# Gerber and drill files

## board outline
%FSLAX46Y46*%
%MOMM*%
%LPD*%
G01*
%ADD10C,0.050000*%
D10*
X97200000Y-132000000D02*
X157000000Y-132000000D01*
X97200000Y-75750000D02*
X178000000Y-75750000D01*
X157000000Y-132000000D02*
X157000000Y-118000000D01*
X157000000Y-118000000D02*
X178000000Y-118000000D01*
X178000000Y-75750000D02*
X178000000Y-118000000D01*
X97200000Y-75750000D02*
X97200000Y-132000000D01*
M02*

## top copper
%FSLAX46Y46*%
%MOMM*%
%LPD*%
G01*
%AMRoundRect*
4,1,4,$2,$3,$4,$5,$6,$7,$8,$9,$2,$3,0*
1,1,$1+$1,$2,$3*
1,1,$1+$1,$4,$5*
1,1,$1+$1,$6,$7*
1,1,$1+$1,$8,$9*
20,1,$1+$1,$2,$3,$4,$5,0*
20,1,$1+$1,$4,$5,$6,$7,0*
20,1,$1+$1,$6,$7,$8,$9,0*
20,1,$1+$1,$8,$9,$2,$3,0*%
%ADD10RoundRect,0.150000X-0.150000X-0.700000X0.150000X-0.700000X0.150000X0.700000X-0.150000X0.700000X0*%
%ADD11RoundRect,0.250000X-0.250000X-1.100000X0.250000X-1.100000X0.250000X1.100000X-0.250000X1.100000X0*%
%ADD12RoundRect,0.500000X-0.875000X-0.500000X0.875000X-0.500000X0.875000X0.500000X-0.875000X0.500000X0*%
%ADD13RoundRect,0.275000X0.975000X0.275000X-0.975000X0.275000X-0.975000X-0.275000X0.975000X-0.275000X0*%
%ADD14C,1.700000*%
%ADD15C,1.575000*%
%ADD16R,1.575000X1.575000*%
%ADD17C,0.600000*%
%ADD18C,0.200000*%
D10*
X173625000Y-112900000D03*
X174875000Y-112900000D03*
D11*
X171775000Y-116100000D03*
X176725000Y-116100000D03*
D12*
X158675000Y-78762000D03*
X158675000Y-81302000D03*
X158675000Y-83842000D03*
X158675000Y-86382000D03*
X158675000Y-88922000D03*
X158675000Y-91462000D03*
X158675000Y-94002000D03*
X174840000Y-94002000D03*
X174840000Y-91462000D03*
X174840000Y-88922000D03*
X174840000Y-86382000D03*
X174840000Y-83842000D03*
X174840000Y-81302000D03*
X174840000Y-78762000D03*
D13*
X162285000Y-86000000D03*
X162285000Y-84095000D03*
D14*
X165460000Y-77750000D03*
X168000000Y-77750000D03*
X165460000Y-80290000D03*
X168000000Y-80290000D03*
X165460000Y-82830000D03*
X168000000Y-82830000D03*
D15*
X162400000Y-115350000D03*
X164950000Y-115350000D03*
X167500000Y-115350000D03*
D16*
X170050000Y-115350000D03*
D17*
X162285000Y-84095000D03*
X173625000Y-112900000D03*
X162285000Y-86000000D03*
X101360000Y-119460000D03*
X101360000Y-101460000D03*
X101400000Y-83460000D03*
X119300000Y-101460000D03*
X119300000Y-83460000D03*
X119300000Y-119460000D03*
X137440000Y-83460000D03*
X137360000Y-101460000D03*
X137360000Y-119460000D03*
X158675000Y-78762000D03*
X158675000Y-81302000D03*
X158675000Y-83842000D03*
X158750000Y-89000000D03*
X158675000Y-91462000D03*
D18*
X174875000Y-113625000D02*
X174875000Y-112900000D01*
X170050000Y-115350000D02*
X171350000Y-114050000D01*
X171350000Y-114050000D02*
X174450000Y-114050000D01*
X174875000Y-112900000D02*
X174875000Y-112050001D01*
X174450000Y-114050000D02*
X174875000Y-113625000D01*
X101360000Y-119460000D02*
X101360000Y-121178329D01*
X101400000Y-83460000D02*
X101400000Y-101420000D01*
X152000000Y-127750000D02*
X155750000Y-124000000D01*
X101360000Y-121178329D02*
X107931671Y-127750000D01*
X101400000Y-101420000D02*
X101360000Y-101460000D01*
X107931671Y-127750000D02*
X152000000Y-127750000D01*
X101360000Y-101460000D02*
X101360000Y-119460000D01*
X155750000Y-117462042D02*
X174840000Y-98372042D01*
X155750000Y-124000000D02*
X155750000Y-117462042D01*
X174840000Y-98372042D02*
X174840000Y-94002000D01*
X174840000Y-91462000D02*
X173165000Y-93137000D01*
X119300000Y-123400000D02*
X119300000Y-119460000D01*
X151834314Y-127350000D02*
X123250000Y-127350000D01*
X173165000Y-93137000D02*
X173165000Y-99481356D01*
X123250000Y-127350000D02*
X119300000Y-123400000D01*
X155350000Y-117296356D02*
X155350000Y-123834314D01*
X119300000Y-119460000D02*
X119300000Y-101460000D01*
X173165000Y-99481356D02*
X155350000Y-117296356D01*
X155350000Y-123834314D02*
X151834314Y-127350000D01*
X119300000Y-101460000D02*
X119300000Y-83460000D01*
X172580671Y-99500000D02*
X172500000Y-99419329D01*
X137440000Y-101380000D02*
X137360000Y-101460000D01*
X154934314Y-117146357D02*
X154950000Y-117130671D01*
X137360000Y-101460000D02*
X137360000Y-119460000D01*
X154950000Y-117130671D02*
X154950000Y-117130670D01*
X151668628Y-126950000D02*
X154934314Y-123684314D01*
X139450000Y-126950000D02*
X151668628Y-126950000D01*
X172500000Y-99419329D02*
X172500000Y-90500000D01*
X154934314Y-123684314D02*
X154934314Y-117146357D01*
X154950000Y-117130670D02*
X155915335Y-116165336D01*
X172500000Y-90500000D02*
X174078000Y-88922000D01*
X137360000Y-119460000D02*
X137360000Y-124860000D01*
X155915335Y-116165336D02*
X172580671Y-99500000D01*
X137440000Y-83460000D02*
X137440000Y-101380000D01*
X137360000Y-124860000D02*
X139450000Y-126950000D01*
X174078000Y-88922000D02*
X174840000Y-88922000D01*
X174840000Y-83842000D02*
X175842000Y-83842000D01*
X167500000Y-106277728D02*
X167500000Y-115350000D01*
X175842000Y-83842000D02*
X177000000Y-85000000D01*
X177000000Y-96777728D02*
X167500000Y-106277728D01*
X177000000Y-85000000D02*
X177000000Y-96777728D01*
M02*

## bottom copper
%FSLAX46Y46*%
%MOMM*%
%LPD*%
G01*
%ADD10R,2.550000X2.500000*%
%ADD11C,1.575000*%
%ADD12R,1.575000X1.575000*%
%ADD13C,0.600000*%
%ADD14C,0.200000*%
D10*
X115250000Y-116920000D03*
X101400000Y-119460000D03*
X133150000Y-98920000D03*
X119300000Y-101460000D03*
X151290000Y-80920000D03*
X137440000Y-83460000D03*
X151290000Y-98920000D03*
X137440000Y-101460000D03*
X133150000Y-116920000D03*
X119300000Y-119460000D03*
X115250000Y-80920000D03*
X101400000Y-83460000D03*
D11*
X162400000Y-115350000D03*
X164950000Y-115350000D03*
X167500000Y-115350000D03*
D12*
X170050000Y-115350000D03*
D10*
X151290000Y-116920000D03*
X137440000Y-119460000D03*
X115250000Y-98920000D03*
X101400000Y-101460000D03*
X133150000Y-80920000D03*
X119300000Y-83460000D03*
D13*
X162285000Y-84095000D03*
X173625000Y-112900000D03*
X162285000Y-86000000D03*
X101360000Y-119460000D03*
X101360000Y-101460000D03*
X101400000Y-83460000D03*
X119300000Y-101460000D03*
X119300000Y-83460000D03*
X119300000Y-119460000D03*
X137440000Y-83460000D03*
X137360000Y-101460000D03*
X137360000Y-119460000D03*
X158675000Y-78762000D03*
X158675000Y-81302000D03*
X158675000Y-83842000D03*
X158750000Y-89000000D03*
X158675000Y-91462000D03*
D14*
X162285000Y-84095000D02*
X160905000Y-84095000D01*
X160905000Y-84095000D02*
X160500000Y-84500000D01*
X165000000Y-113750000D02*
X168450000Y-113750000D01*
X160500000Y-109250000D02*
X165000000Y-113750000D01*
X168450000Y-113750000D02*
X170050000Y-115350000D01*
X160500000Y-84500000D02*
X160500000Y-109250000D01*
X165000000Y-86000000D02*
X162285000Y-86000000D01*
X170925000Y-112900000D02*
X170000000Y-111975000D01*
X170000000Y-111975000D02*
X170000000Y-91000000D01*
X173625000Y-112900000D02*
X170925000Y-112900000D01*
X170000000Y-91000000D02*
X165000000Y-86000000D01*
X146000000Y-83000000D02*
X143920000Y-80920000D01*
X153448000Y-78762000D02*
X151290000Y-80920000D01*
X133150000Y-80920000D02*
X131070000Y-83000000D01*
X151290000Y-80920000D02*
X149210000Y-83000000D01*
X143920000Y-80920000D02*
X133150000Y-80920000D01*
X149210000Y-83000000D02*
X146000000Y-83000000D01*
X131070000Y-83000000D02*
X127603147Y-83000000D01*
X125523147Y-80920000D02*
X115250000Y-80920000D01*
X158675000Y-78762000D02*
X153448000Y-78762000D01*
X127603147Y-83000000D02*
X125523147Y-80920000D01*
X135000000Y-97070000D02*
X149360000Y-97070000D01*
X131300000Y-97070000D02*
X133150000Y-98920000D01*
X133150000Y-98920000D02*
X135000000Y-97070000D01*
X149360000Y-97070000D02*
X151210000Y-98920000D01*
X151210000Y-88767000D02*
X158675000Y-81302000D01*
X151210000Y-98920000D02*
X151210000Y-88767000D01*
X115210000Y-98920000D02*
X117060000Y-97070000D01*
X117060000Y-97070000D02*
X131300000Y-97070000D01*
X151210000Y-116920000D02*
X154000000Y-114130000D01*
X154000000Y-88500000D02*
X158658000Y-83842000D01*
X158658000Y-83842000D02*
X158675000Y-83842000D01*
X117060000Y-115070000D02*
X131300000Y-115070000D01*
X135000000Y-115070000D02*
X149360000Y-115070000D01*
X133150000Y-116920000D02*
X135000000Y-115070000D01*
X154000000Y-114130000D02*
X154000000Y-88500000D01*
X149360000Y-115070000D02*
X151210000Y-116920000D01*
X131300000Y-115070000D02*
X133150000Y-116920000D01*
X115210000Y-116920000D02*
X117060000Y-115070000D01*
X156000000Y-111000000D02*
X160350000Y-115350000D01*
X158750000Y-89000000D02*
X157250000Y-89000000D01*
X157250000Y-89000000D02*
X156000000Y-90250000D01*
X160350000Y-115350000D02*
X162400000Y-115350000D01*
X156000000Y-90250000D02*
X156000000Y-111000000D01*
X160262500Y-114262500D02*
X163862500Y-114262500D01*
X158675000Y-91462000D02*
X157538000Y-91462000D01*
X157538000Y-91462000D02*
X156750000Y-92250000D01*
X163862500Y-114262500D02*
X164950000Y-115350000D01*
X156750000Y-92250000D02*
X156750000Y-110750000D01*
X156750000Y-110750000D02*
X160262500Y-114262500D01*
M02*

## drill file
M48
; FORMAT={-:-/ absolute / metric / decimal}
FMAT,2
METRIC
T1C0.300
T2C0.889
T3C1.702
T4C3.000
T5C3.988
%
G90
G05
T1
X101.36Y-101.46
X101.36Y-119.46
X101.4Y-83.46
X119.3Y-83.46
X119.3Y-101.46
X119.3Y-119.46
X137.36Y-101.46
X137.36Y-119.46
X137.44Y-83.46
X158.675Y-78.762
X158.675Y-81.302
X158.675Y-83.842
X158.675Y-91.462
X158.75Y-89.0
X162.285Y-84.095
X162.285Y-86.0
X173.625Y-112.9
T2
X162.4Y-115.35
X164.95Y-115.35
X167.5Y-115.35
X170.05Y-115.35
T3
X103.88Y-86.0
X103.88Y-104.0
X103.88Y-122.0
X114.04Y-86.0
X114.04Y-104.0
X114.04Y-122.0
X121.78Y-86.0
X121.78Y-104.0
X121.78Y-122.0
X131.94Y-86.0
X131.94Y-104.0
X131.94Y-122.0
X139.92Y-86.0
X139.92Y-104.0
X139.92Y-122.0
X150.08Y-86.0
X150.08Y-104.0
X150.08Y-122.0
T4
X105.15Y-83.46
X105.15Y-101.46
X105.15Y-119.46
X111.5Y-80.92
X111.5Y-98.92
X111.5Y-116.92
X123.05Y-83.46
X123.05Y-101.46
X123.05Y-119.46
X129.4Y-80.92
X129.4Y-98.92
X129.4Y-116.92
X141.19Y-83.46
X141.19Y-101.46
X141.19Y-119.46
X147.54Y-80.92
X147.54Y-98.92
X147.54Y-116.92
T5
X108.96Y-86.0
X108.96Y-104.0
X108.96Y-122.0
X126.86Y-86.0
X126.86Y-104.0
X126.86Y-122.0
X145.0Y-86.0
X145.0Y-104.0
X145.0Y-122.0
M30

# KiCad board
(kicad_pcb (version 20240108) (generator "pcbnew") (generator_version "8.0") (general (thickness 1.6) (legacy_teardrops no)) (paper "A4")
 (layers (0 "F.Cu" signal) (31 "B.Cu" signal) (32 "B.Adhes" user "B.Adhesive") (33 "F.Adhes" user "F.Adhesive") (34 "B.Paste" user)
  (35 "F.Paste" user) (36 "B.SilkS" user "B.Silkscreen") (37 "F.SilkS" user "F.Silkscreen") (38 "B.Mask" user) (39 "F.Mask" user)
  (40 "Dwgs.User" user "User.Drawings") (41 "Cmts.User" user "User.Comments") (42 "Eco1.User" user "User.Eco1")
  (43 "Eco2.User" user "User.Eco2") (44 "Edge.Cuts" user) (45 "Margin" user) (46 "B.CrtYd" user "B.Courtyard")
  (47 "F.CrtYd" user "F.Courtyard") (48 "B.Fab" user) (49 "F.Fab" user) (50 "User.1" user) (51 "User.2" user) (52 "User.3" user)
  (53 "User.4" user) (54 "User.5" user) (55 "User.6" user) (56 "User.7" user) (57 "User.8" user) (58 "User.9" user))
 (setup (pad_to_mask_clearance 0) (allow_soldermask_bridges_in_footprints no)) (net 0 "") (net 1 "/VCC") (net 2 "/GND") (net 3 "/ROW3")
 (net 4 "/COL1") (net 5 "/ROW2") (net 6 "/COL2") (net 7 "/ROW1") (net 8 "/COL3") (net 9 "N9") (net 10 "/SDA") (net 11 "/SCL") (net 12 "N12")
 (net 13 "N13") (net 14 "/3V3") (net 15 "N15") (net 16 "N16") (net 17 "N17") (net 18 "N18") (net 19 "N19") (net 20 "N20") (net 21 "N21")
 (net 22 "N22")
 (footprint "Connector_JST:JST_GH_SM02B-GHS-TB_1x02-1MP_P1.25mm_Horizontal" (layer "F.Cu") (at 174.25 114.75)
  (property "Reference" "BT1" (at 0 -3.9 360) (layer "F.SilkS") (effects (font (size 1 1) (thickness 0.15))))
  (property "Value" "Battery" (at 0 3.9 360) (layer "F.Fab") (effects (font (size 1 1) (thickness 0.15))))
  (pad "1" smd roundrect (at -0.625 -1.85) (size 0.6 1.7) (layers "F.Cu" "F.Paste" "F.Mask") (roundrect_rratio 0.25) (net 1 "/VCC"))
  (pad "2" smd roundrect (at 0.625 -1.85) (size 0.6 1.7) (layers "F.Cu" "F.Paste" "F.Mask") (roundrect_rratio 0.25) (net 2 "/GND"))
  (pad "MP" smd roundrect (at -2.475 1.35) (size 1 2.7) (layers "F.Cu" "F.Paste" "F.Mask") (roundrect_rratio 0.25))
  (pad "MP" smd roundrect (at 2.475 1.35) (size 1 2.7) (layers "F.Cu" "F.Paste" "F.Mask") (roundrect_rratio 0.25)))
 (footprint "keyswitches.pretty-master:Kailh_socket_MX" (layer "F.Cu") (at 108.96 122)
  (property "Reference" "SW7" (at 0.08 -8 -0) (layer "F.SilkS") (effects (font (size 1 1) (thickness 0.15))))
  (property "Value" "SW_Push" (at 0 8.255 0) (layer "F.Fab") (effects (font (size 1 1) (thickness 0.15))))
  (pad "" np_thru_hole circle (at -5.08 0) (size 1.7018 1.7018) (drill 1.7018) (layers "*.Cu" "*.Mask"))
  (pad "" np_thru_hole circle (at -3.81 -2.54) (size 3 3) (drill 3) (layers "*.Cu" "*.Mask"))
  (pad "" np_thru_hole circle (at 0 0) (size 3.9878 3.9878) (drill 3.9878) (layers "*.Cu" "*.Mask"))
  (pad "" np_thru_hole circle (at 2.54 -5.08) (size 3 3) (drill 3) (layers "*.Cu" "*.Mask"))
  (pad "" np_thru_hole circle (at 5.08 0) (size 1.7018 1.7018) (drill 1.7018) (layers "*.Cu" "*.Mask"))
  (pad "1" smd rect (at 6.29 -5.08) (size 2.55 2.5) (layers "B.Cu" "B.Paste" "B.Mask") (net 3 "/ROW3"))
  (pad "2" smd rect (at -7.56 -2.54) (size 2.55 2.5) (layers "B.Cu" "B.Paste" "B.Mask") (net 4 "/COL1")))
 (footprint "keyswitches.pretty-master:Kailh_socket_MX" (layer "F.Cu") (at 126.86 104)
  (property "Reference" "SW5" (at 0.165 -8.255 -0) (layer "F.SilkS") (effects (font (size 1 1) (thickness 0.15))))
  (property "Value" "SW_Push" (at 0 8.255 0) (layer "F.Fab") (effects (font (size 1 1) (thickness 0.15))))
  (pad "" np_thru_hole circle (at -5.08 0) (size 1.7018 1.7018) (drill 1.7018) (layers "*.Cu" "*.Mask"))
  (pad "" np_thru_hole circle (at -3.81 -2.54) (size 3 3) (drill 3) (layers "*.Cu" "*.Mask"))
  (pad "" np_thru_hole circle (at 0 0) (size 3.9878 3.9878) (drill 3.9878) (layers "*.Cu" "*.Mask"))
  (pad "" np_thru_hole circle (at 2.54 -5.08) (size 3 3) (drill 3) (layers "*.Cu" "*.Mask"))
  (pad "" np_thru_hole circle (at 5.08 0) (size 1.7018 1.7018) (drill 1.7018) (layers "*.Cu" "*.Mask"))
  (pad "1" smd rect (at 6.29 -5.08) (size 2.55 2.5) (layers "B.Cu" "B.Paste" "B.Mask") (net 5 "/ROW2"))
  (pad "2" smd rect (at -7.56 -2.54) (size 2.55 2.5) (layers "B.Cu" "B.Paste" "B.Mask") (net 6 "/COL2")))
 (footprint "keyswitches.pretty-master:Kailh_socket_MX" (layer "F.Cu") (at 145 86)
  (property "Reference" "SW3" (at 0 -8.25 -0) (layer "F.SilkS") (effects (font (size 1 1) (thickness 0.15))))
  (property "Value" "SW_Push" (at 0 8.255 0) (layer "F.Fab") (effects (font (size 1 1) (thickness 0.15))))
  (pad "" np_thru_hole circle (at -5.08 0) (size 1.7018 1.7018) (drill 1.7018) (layers "*.Cu" "*.Mask"))
  (pad "" np_thru_hole circle (at -3.81 -2.54) (size 3 3) (drill 3) (layers "*.Cu" "*.Mask"))
  (pad "" np_thru_hole circle (at 0 0) (size 3.9878 3.9878) (drill 3.9878) (layers "*.Cu" "*.Mask"))
  (pad "" np_thru_hole circle (at 2.54 -5.08) (size 3 3) (drill 3) (layers "*.Cu" "*.Mask"))
  (pad "" np_thru_hole circle (at 5.08 0) (size 1.7018 1.7018) (drill 1.7018) (layers "*.Cu" "*.Mask"))
  (pad "1" smd rect (at 6.29 -5.08) (size 2.55 2.5) (layers "B.Cu" "B.Paste" "B.Mask") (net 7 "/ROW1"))
  (pad "2" smd rect (at -7.56 -2.54) (size 2.55 2.5) (layers "B.Cu" "B.Paste" "B.Mask") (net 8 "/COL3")))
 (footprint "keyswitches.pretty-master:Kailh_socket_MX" (layer "F.Cu") (at 145 104)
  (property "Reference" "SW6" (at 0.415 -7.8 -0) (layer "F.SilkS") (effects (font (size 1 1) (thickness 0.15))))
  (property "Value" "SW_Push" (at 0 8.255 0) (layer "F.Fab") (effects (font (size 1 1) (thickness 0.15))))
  (pad "" np_thru_hole circle (at -5.08 0) (size 1.7018 1.7018) (drill 1.7018) (layers "*.Cu" "*.Mask"))
  (pad "" np_thru_hole circle (at -3.81 -2.54) (size 3 3) (drill 3) (layers "*.Cu" "*.Mask"))
  (pad "" np_thru_hole circle (at 0 0) (size 3.9878 3.9878) (drill 3.9878) (layers "*.Cu" "*.Mask"))
  (pad "" np_thru_hole circle (at 2.54 -5.08) (size 3 3) (drill 3) (layers "*.Cu" "*.Mask"))
  (pad "" np_thru_hole circle (at 5.08 0) (size 1.7018 1.7018) (drill 1.7018) (layers "*.Cu" "*.Mask"))
  (pad "1" smd rect (at 6.29 -5.08) (size 2.55 2.5) (layers "B.Cu" "B.Paste" "B.Mask") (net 5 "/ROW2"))
  (pad "2" smd rect (at -7.56 -2.54) (size 2.55 2.5) (layers "B.Cu" "B.Paste" "B.Mask") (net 8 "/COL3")))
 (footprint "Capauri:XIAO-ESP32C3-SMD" (layer "F.Cu") (at 166.675 86.342)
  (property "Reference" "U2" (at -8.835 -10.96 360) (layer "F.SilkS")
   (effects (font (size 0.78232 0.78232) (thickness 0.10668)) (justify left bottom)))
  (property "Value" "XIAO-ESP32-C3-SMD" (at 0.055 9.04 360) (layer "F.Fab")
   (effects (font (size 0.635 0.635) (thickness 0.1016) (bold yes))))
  (pad "1" smd roundrect (at -8 -7.58) (size 2.75 2) (layers "F.Cu" "F.Paste" "F.Mask") (roundrect_rratio 0.25) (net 7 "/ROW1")
   (solder_mask_margin 0.0508) (thermal_bridge_angle 45))
  (pad "2" smd roundrect (at -8 -5.04) (size 2.75 2) (layers "F.Cu" "F.Paste" "F.Mask") (roundrect_rratio 0.25) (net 5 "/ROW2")
   (solder_mask_margin 0.0508) (thermal_bridge_angle 45))
  (pad "3" smd roundrect (at -8 -2.5) (size 2.75 2) (layers "F.Cu" "F.Paste" "F.Mask") (roundrect_rratio 0.25) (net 3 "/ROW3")
   (solder_mask_margin 0.0508) (thermal_bridge_angle 45))
  (pad "4" smd roundrect (at -8 0.04) (size 2.75 2) (layers "F.Cu" "F.Paste" "F.Mask") (roundrect_rratio 0.25) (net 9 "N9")
   (solder_mask_margin 0.0508) (thermal_bridge_angle 45))
  (pad "5" smd roundrect (at -8 2.58) (size 2.75 2) (layers "F.Cu" "F.Paste" "F.Mask") (roundrect_rratio 0.25) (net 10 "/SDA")
   (solder_mask_margin 0.0508) (thermal_bridge_angle 45))
  (pad "6" smd roundrect (at -8 5.12) (size 2.75 2) (layers "F.Cu" "F.Paste" "F.Mask") (roundrect_rratio 0.25) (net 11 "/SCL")
   (solder_mask_margin 0.0508) (thermal_bridge_angle 45))
  (pad "7" smd roundrect (at -8 7.66) (size 2.75 2) (layers "F.Cu" "F.Paste" "F.Mask") (roundrect_rratio 0.25) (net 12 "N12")
   (solder_mask_margin 0.0508) (thermal_bridge_angle 45))
  (pad "8" smd roundrect (at 8.165 7.66) (size 2.75 2) (layers "F.Cu" "F.Paste" "F.Mask") (roundrect_rratio 0.25) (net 4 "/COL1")
   (solder_mask_margin 0.0508) (thermal_bridge_angle 45))
  (pad "9" smd roundrect (at 8.165 5.12) (size 2.75 2) (layers "F.Cu" "F.Paste" "F.Mask") (roundrect_rratio 0.25) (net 6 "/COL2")
   (solder_mask_margin 0.0508) (thermal_bridge_angle 45))
  (pad "10" smd roundrect (at 8.165 2.58) (size 2.75 2) (layers "F.Cu" "F.Paste" "F.Mask") (roundrect_rratio 0.25) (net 8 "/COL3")
   (solder_mask_margin 0.0508) (thermal_bridge_angle 45))
  (pad "11" smd roundrect (at 8.165 0.04) (size 2.75 2) (layers "F.Cu" "F.Paste" "F.Mask") (roundrect_rratio 0.25) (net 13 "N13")
   (solder_mask_margin 0.0508) (thermal_bridge_angle 45))
  (pad "12" smd roundrect (at 8.165 -2.5) (size 2.75 2) (layers "F.Cu" "F.Paste" "F.Mask") (roundrect_rratio 0.25) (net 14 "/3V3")
   (solder_mask_margin 0.0508) (thermal_bridge_angle 45))
  (pad "13" smd roundrect (at 8.165 -5.04) (size 2.75 2) (layers "F.Cu" "F.Paste" "F.Mask") (roundrect_rratio 0.25) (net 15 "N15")
   (solder_mask_margin 0.0508) (thermal_bridge_angle 45))
  (pad "14" smd roundrect (at 8.165 -7.58) (size 2.75 2) (layers "F.Cu" "F.Paste" "F.Mask") (roundrect_rratio 0.25) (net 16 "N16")
   (solder_mask_margin 0.0508) (thermal_bridge_angle 45))
  (pad "15" smd roundrect (at -4.39 -0.342 180) (size 2.5 1.1) (layers "F.Cu" "F.Paste" "F.Mask") (roundrect_rratio 0.25) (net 1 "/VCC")
   (solder_mask_margin 0.0508) (thermal_bridge_angle 45))
  (pad "16" smd roundrect (at -4.39 -2.247 180) (size 2.5 1.1) (layers "F.Cu" "F.Paste" "F.Mask") (roundrect_rratio 0.25) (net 2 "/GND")
   (solder_mask_margin 0.0508) (thermal_bridge_angle 45))
  (pad "17" smd circle (at -1.215 -8.592) (size 1.7 1.7) (layers "F.Cu" "F.Paste" "F.Mask") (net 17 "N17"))
  (pad "18" smd circle (at 1.325 -8.592) (size 1.7 1.7) (layers "F.Cu" "F.Paste" "F.Mask") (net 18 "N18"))
  (pad "19" smd circle (at -1.215 -6.052) (size 1.7 1.7) (layers "F.Cu" "F.Paste" "F.Mask") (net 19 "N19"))
  (pad "20" smd circle (at 1.325 -6.052) (size 1.7 1.7) (layers "F.Cu" "F.Paste" "F.Mask") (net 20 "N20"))
  (pad "21" smd circle (at -1.215 -3.512) (size 1.7 1.7) (layers "F.Cu" "F.Paste" "F.Mask") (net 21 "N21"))
  (pad "22" smd circle (at 1.325 -3.512) (size 1.7 1.7) (layers "F.Cu" "F.Paste" "F.Mask") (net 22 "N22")))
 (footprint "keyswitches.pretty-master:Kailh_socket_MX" (layer "F.Cu") (at 126.86 122)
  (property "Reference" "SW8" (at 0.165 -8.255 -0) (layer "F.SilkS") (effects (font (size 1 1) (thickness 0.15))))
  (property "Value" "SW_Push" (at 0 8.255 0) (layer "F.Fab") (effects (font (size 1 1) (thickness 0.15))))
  (pad "" np_thru_hole circle (at -5.08 0) (size 1.7018 1.7018) (drill 1.7018) (layers "*.Cu" "*.Mask"))
  (pad "" np_thru_hole circle (at -3.81 -2.54) (size 3 3) (drill 3) (layers "*.Cu" "*.Mask"))
  (pad "" np_thru_hole circle (at 0 0) (size 3.9878 3.9878) (drill 3.9878) (layers "*.Cu" "*.Mask"))
  (pad "" np_thru_hole circle (at 2.54 -5.08) (size 3 3) (drill 3) (layers "*.Cu" "*.Mask"))
  (pad "" np_thru_hole circle (at 5.08 0) (size 1.7018 1.7018) (drill 1.7018) (layers "*.Cu" "*.Mask"))
  (pad "1" smd rect (at 6.29 -5.08) (size 2.55 2.5) (layers "B.Cu" "B.Paste" "B.Mask") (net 3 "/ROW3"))
  (pad "2" smd rect (at -7.56 -2.54) (size 2.55 2.5) (layers "B.Cu" "B.Paste" "B.Mask") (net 6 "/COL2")))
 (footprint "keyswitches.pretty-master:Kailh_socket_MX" (layer "F.Cu") (at 108.96 86)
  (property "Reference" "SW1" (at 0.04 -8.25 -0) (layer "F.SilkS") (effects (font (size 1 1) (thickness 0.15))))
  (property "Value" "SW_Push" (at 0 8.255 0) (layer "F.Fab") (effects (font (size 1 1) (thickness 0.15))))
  (pad "" np_thru_hole circle (at -5.08 0) (size 1.7018 1.7018) (drill 1.7018) (layers "*.Cu" "*.Mask"))
  (pad "" np_thru_hole circle (at -3.81 -2.54) (size 3 3) (drill 3) (layers "*.Cu" "*.Mask"))
  (pad "" np_thru_hole circle (at 0 0) (size 3.9878 3.9878) (drill 3.9878) (layers "*.Cu" "*.Mask"))
  (pad "" np_thru_hole circle (at 2.54 -5.08) (size 3 3) (drill 3) (layers "*.Cu" "*.Mask"))
  (pad "" np_thru_hole circle (at 5.08 0) (size 1.7018 1.7018) (drill 1.7018) (layers "*.Cu" "*.Mask"))
  (pad "1" smd rect (at 6.29 -5.08) (size 2.55 2.5) (layers "B.Cu" "B.Paste" "B.Mask") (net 7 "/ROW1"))
  (pad "2" smd rect (at -7.56 -2.54) (size 2.55 2.5) (layers "B.Cu" "B.Paste" "B.Mask") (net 4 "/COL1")))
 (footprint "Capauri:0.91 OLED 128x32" (layer "F.Cu") (at 166.25 121.9)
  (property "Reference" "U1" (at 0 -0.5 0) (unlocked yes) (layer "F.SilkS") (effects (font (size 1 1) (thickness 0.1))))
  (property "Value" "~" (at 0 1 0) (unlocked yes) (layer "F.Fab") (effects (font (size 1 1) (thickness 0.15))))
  (pad "1" thru_hole circle (at -3.85 -6.55) (size 1.575 1.575) (drill 0.889) (layers "*.Cu" "*.Mask") (remove_unused_layers no)
   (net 10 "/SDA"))
  (pad "2" thru_hole circle (at -1.3 -6.55) (size 1.575 1.575) (drill 0.889) (layers "*.Cu" "*.Mask") (remove_unused_layers no)
   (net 11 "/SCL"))
  (pad "3" thru_hole circle (at 1.25 -6.55) (size 1.575 1.575) (drill 0.889) (layers "*.Cu" "*.Mask") (remove_unused_layers no)
   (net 14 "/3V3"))
  (pad "4" thru_hole rect (at 3.8 -6.55) (size 1.575 1.575) (drill 0.889) (layers "*.Cu" "*.Mask") (remove_unused_layers no) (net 2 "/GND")
   (thermal_bridge_angle 45)))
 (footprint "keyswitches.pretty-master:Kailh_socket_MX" (layer "F.Cu") (at 145 122)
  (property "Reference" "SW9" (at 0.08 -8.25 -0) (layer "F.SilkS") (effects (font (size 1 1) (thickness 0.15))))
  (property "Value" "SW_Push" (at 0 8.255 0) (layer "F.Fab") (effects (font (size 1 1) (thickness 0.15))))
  (pad "" np_thru_hole circle (at -5.08 0) (size 1.7018 1.7018) (drill 1.7018) (layers "*.Cu" "*.Mask"))
  (pad "" np_thru_hole circle (at -3.81 -2.54) (size 3 3) (drill 3) (layers "*.Cu" "*.Mask"))
  (pad "" np_thru_hole circle (at 0 0) (size 3.9878 3.9878) (drill 3.9878) (layers "*.Cu" "*.Mask"))
  (pad "" np_thru_hole circle (at 2.54 -5.08) (size 3 3) (drill 3) (layers "*.Cu" "*.Mask"))
  (pad "" np_thru_hole circle (at 5.08 0) (size 1.7018 1.7018) (drill 1.7018) (layers "*.Cu" "*.Mask"))
  (pad "1" smd rect (at 6.29 -5.08) (size 2.55 2.5) (layers "B.Cu" "B.Paste" "B.Mask") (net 3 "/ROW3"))
  (pad "2" smd rect (at -7.56 -2.54) (size 2.55 2.5) (layers "B.Cu" "B.Paste" "B.Mask") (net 8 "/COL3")))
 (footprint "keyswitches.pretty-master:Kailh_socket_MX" (layer "F.Cu") (at 108.96 104)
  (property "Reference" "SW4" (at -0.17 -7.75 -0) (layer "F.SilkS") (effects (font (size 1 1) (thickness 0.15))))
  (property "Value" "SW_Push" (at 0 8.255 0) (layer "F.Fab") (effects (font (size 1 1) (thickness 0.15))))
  (pad "" np_thru_hole circle (at -5.08 0) (size 1.7018 1.7018) (drill 1.7018) (layers "*.Cu" "*.Mask"))
  (pad "" np_thru_hole circle (at -3.81 -2.54) (size 3 3) (drill 3) (layers "*.Cu" "*.Mask"))
  (pad "" np_thru_hole circle (at 0 0) (size 3.9878 3.9878) (drill 3.9878) (layers "*.Cu" "*.Mask"))
  (pad "" np_thru_hole circle (at 2.54 -5.08) (size 3 3) (drill 3) (layers "*.Cu" "*.Mask"))
  (pad "" np_thru_hole circle (at 5.08 0) (size 1.7018 1.7018) (drill 1.7018) (layers "*.Cu" "*.Mask"))
  (pad "1" smd rect (at 6.29 -5.08) (size 2.55 2.5) (layers "B.Cu" "B.Paste" "B.Mask") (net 5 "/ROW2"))
  (pad "2" smd rect (at -7.56 -2.54) (size 2.55 2.5) (layers "B.Cu" "B.Paste" "B.Mask") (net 4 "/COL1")))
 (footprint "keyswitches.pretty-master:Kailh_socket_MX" (layer "F.Cu") (at 126.86 86)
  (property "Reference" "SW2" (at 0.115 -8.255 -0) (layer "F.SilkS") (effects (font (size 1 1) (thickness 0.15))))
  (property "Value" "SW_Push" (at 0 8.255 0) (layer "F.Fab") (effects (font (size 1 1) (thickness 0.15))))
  (pad "" np_thru_hole circle (at -5.08 0) (size 1.7018 1.7018) (drill 1.7018) (layers "*.Cu" "*.Mask"))
  (pad "" np_thru_hole circle (at -3.81 -2.54) (size 3 3) (drill 3) (layers "*.Cu" "*.Mask"))
  (pad "" np_thru_hole circle (at 0 0) (size 3.9878 3.9878) (drill 3.9878) (layers "*.Cu" "*.Mask"))
  (pad "" np_thru_hole circle (at 2.54 -5.08) (size 3 3) (drill 3) (layers "*.Cu" "*.Mask"))
  (pad "" np_thru_hole circle (at 5.08 0) (size 1.7018 1.7018) (drill 1.7018) (layers "*.Cu" "*.Mask"))
  (pad "1" smd rect (at 6.29 -5.08) (size 2.55 2.5) (layers "B.Cu" "B.Paste" "B.Mask") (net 7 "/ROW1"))
  (pad "2" smd rect (at -7.56 -2.54) (size 2.55 2.5) (layers "B.Cu" "B.Paste" "B.Mask") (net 6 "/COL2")))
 (gr_line (start 97.2 132) (end 157 132) (stroke (width 0.05) (type default)) (layer "Edge.Cuts"))
 (gr_line (start 97.2 75.75) (end 178 75.75) (stroke (width 0.05) (type default)) (layer "Edge.Cuts"))
 (gr_line (start 157 132) (end 157 118) (stroke (width 0.05) (type default)) (layer "Edge.Cuts"))
 (gr_line (start 157 118) (end 178 118) (stroke (width 0.05) (type default)) (layer "Edge.Cuts"))
 (gr_line (start 178 75.75) (end 178 118) (stroke (width 0.05) (type default)) (layer "Edge.Cuts"))
 (gr_line (start 97.2 75.75) (end 97.2 132) (stroke (width 0.05) (type default)) (layer "Edge.Cuts"))
 (segment (start 174.875 113.625) (end 174.875 112.9) (width 0.2) (layer "F.Cu") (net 2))
 (segment (start 170.05 115.35) (end 171.35 114.05) (width 0.2) (layer "F.Cu") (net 2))
 (segment (start 171.35 114.05) (end 174.45 114.05) (width 0.2) (layer "F.Cu") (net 2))
 (segment (start 174.875 112.9) (end 174.875 112.050001) (width 0.2) (layer "F.Cu") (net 2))
 (segment (start 174.45 114.05) (end 174.875 113.625) (width 0.2) (layer "F.Cu") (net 2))
 (via (at 162.285 84.095) (size 0.6) (drill 0.3) (layers "F.Cu" "B.Cu") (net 2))
 (segment (start 162.285 84.095) (end 160.905 84.095) (width 0.2) (layer "B.Cu") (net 2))
 (segment (start 160.905 84.095) (end 160.5 84.5) (width 0.2) (layer "B.Cu") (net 2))
 (segment (start 165 113.75) (end 168.45 113.75) (width 0.2) (layer "B.Cu") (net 2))
 (segment (start 160.5 109.25) (end 165 113.75) (width 0.2) (layer "B.Cu") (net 2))
 (segment (start 168.45 113.75) (end 170.05 115.35) (width 0.2) (layer "B.Cu") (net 2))
 (segment (start 160.5 84.5) (end 160.5 109.25) (width 0.2) (layer "B.Cu") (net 2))
 (via (at 173.625 112.9) (size 0.6) (drill 0.3) (layers "F.Cu" "B.Cu") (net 1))
 (via (at 162.285 86) (size 0.6) (drill 0.3) (layers "F.Cu" "B.Cu") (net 1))
 (segment (start 165 86) (end 162.285 86) (width 0.2) (layer "B.Cu") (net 1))
 (segment (start 170.925 112.9) (end 170 111.975) (width 0.2) (layer "B.Cu") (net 1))
 (segment (start 170 111.975) (end 170 91) (width 0.2) (layer "B.Cu") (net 1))
 (segment (start 173.625 112.9) (end 170.925 112.9) (width 0.2) (layer "B.Cu") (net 1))
 (segment (start 170 91) (end 165 86) (width 0.2) (layer "B.Cu") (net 1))
 (segment (start 101.36 119.46) (end 101.36 121.178329) (width 0.2) (layer "F.Cu") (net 4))
 (segment (start 101.4 83.46) (end 101.4 101.42) (width 0.2) (layer "F.Cu") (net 4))
 (segment (start 152 127.75) (end 155.75 124) (width 0.2) (layer "F.Cu") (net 4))
 (segment (start 101.36 121.178329) (end 107.931671 127.75) (width 0.2) (layer "F.Cu") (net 4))
 (segment (start 101.4 101.42) (end 101.36 101.46) (width 0.2) (layer "F.Cu") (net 4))
 (segment (start 107.931671 127.75) (end 152 127.75) (width 0.2) (layer "F.Cu") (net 4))
 (segment (start 101.36 101.46) (end 101.36 119.46) (width 0.2) (layer "F.Cu") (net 4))
 (segment (start 155.75 117.462042) (end 174.84 98.372042) (width 0.2) (layer "F.Cu") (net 4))
 (segment (start 155.75 124) (end 155.75 117.462042) (width 0.2) (layer "F.Cu") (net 4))
 (segment (start 174.84 98.372042) (end 174.84 94.002) (width 0.2) (layer "F.Cu") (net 4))
 (via (at 101.36 119.46) (size 0.6) (drill 0.3) (layers "F.Cu" "B.Cu") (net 4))
 (via (at 101.36 101.46) (size 0.6) (drill 0.3) (layers "F.Cu" "B.Cu") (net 4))
 (via (at 101.4 83.46) (size 0.6) (drill 0.3) (layers "F.Cu" "B.Cu") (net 4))
 (segment (start 174.84 91.462) (end 173.165 93.137) (width 0.2) (layer "F.Cu") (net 6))
 (segment (start 119.3 123.4) (end 119.3 119.46) (width 0.2) (layer "F.Cu") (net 6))
 (segment (start 151.834314 127.35) (end 123.25 127.35) (width 0.2) (layer "F.Cu") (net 6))
 (segment (start 173.165 93.137) (end 173.165 99.481356) (width 0.2) (layer "F.Cu") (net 6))
 (segment (start 123.25 127.35) (end 119.3 123.4) (width 0.2) (layer "F.Cu") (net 6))
 (segment (start 155.35 117.296356) (end 155.35 123.834314) (width 0.2) (layer "F.Cu") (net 6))
 (segment (start 119.3 119.46) (end 119.3 101.46) (width 0.2) (layer "F.Cu") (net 6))
 (segment (start 173.165 99.481356) (end 155.35 117.296356) (width 0.2) (layer "F.Cu") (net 6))
 (segment (start 155.35 123.834314) (end 151.834314 127.35) (width 0.2) (layer "F.Cu") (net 6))
 (segment (start 119.3 101.46) (end 119.3 83.46) (width 0.2) (layer "F.Cu") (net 6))
 (via (at 119.3 101.46) (size 0.6) (drill 0.3) (layers "F.Cu" "B.Cu") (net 6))
 (via (at 119.3 83.46) (size 0.6) (drill 0.3) (layers "F.Cu" "B.Cu") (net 6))
 (via (at 119.3 119.46) (size 0.6) (drill 0.3) (layers "F.Cu" "B.Cu") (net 6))
 (segment (start 172.580671 99.5) (end 172.5 99.419329) (width 0.2) (layer "F.Cu") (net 8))
 (segment (start 137.44 101.38) (end 137.36 101.46) (width 0.2) (layer "F.Cu") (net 8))
 (segment (start 154.934314 117.146357) (end 154.95 117.130671) (width 0.2) (layer "F.Cu") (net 8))
 (segment (start 137.36 101.46) (end 137.36 119.46) (width 0.2) (layer "F.Cu") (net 8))
 (segment (start 154.95 117.130671) (end 154.95 117.13067) (width 0.2) (layer "F.Cu") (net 8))
 (segment (start 151.668628 126.95) (end 154.934314 123.684314) (width 0.2) (layer "F.Cu") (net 8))
 (segment (start 139.45 126.95) (end 151.668628 126.95) (width 0.2) (layer "F.Cu") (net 8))
 (segment (start 172.5 99.419329) (end 172.5 90.5) (width 0.2) (layer "F.Cu") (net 8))
 (segment (start 154.934314 123.684314) (end 154.934314 117.146357) (width 0.2) (layer "F.Cu") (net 8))
 (segment (start 154.95 117.13067) (end 155.915335 116.165336) (width 0.2) (layer "F.Cu") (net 8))
 (segment (start 172.5 90.5) (end 174.078 88.922) (width 0.2) (layer "F.Cu") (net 8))
 (segment (start 137.36 119.46) (end 137.36 124.86) (width 0.2) (layer "F.Cu") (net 8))
 (segment (start 155.915335 116.165336) (end 172.580671 99.5) (width 0.2) (layer "F.Cu") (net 8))
 (segment (start 137.44 83.46) (end 137.44 101.38) (width 0.2) (layer "F.Cu") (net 8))
 (segment (start 137.36 124.86) (end 139.45 126.95) (width 0.2) (layer "F.Cu") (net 8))
 (segment (start 174.078 88.922) (end 174.84 88.922) (width 0.2) (layer "F.Cu") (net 8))
 (via (at 137.44 83.46) (size 0.6) (drill 0.3) (layers "F.Cu" "B.Cu") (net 8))
 (via (at 137.36 101.46) (size 0.6) (drill 0.3) (layers "F.Cu" "B.Cu") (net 8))
 (via (at 137.36 119.46) (size 0.6) (drill 0.3) (layers "F.Cu" "B.Cu") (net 8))
 (segment (start 174.84 83.842) (end 175.842 83.842) (width 0.2) (layer "F.Cu") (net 14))
 (segment (start 167.5 106.277728) (end 167.5 115.35) (width 0.2) (layer "F.Cu") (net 14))
 (segment (start 175.842 83.842) (end 177 85) (width 0.2) (layer "F.Cu") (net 14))
 (segment (start 177 96.777728) (end 167.5 106.277728) (width 0.2) (layer "F.Cu") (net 14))
 (segment (start 177 85) (end 177 96.777728) (width 0.2) (layer "F.Cu") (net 14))
 (via (at 158.675 78.762) (size 0.6) (drill 0.3) (layers "F.Cu" "B.Cu") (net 7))
 (segment (start 146 83) (end 143.92 80.92) (width 0.2) (layer "B.Cu") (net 7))
 (segment (start 153.448 78.762) (end 151.29 80.92) (width 0.2) (layer "B.Cu") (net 7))
 (segment (start 133.15 80.92) (end 131.07 83) (width 0.2) (layer "B.Cu") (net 7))
 (segment (start 151.29 80.92) (end 149.21 83) (width 0.2) (layer "B.Cu") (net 7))
 (segment (start 143.92 80.92) (end 133.15 80.92) (width 0.2) (layer "B.Cu") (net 7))
 (segment (start 149.21 83) (end 146 83) (width 0.2) (layer "B.Cu") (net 7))
 (segment (start 131.07 83) (end 127.603147 83) (width 0.2) (layer "B.Cu") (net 7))
 (segment (start 125.523147 80.92) (end 115.25 80.92) (width 0.2) (layer "B.Cu") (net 7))
 (segment (start 158.675 78.762) (end 153.448 78.762) (width 0.2) (layer "B.Cu") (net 7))
 (segment (start 127.603147 83) (end 125.523147 80.92) (width 0.2) (layer "B.Cu") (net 7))
 (via (at 158.675 81.302) (size 0.6) (drill 0.3) (layers "F.Cu" "B.Cu") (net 5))
 (segment (start 135 97.07) (end 149.36 97.07) (width 0.2) (layer "B.Cu") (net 5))
 (segment (start 131.3 97.07) (end 133.15 98.92) (width 0.2) (layer "B.Cu") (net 5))
 (segment (start 133.15 98.92) (end 135 97.07) (width 0.2) (layer "B.Cu") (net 5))
 (segment (start 149.36 97.07) (end 151.21 98.92) (width 0.2) (layer "B.Cu") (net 5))
 (segment (start 151.21 88.767) (end 158.675 81.302) (width 0.2) (layer "B.Cu") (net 5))
 (segment (start 151.21 98.92) (end 151.21 88.767) (width 0.2) (layer "B.Cu") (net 5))
 (segment (start 115.21 98.92) (end 117.06 97.07) (width 0.2) (layer "B.Cu") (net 5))
 (segment (start 117.06 97.07) (end 131.3 97.07) (width 0.2) (layer "B.Cu") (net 5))
 (via (at 158.675 83.842) (size 0.6) (drill 0.3) (layers "F.Cu" "B.Cu") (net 3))
 (segment (start 151.21 116.92) (end 154 114.13) (width 0.2) (layer "B.Cu") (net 3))
 (segment (start 154 88.5) (end 158.658 83.842) (width 0.2) (layer "B.Cu") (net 3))
 (segment (start 158.658 83.842) (end 158.675 83.842) (width 0.2) (layer "B.Cu") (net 3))
 (segment (start 117.06 115.07) (end 131.3 115.07) (width 0.2) (layer "B.Cu") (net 3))
 (segment (start 135 115.07) (end 149.36 115.07) (width 0.2) (layer "B.Cu") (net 3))
 (segment (start 133.15 116.92) (end 135 115.07) (width 0.2) (layer "B.Cu") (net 3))
 (segment (start 154 114.13) (end 154 88.5) (width 0.2) (layer "B.Cu") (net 3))
 (segment (start 149.36 115.07) (end 151.21 116.92) (width 0.2) (layer "B.Cu") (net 3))
 (segment (start 131.3 115.07) (end 133.15 116.92) (width 0.2) (layer "B.Cu") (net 3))
 (segment (start 115.21 116.92) (end 117.06 115.07) (width 0.2) (layer "B.Cu") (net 3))
 (via (at 158.75 89) (size 0.6) (drill 0.3) (layers "F.Cu" "B.Cu") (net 10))
 (segment (start 156 111) (end 160.35 115.35) (width 0.2) (layer "B.Cu") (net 10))
 (segment (start 158.75 89) (end 157.25 89) (width 0.2) (layer "B.Cu") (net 10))
 (segment (start 157.25 89) (end 156 90.25) (width 0.2) (layer "B.Cu") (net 10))
 (segment (start 160.35 115.35) (end 162.4 115.35) (width 0.2) (layer "B.Cu") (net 10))
 (segment (start 156 90.25) (end 156 111) (width 0.2) (layer "B.Cu") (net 10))
 (via (at 158.675 91.462) (size 0.6) (drill 0.3) (layers "F.Cu" "B.Cu") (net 11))
 (segment (start 160.2625 114.2625) (end 163.8625 114.2625) (width 0.2) (layer "B.Cu") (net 11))
 (segment (start 158.675 91.462) (end 157.538 91.462) (width 0.2) (layer "B.Cu") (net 11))
 (segment (start 157.538 91.462) (end 156.75 92.25) (width 0.2) (layer "B.Cu") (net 11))
 (segment (start 163.8625 114.2625) (end 164.95 115.35) (width 0.2) (layer "B.Cu") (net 11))
 (segment (start 156.75 92.25) (end 156.75 110.75) (width 0.2) (layer "B.Cu") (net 11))
 (segment (start 156.75 110.75) (end 160.2625 114.2625) (width 0.2) (layer "B.Cu") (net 11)))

